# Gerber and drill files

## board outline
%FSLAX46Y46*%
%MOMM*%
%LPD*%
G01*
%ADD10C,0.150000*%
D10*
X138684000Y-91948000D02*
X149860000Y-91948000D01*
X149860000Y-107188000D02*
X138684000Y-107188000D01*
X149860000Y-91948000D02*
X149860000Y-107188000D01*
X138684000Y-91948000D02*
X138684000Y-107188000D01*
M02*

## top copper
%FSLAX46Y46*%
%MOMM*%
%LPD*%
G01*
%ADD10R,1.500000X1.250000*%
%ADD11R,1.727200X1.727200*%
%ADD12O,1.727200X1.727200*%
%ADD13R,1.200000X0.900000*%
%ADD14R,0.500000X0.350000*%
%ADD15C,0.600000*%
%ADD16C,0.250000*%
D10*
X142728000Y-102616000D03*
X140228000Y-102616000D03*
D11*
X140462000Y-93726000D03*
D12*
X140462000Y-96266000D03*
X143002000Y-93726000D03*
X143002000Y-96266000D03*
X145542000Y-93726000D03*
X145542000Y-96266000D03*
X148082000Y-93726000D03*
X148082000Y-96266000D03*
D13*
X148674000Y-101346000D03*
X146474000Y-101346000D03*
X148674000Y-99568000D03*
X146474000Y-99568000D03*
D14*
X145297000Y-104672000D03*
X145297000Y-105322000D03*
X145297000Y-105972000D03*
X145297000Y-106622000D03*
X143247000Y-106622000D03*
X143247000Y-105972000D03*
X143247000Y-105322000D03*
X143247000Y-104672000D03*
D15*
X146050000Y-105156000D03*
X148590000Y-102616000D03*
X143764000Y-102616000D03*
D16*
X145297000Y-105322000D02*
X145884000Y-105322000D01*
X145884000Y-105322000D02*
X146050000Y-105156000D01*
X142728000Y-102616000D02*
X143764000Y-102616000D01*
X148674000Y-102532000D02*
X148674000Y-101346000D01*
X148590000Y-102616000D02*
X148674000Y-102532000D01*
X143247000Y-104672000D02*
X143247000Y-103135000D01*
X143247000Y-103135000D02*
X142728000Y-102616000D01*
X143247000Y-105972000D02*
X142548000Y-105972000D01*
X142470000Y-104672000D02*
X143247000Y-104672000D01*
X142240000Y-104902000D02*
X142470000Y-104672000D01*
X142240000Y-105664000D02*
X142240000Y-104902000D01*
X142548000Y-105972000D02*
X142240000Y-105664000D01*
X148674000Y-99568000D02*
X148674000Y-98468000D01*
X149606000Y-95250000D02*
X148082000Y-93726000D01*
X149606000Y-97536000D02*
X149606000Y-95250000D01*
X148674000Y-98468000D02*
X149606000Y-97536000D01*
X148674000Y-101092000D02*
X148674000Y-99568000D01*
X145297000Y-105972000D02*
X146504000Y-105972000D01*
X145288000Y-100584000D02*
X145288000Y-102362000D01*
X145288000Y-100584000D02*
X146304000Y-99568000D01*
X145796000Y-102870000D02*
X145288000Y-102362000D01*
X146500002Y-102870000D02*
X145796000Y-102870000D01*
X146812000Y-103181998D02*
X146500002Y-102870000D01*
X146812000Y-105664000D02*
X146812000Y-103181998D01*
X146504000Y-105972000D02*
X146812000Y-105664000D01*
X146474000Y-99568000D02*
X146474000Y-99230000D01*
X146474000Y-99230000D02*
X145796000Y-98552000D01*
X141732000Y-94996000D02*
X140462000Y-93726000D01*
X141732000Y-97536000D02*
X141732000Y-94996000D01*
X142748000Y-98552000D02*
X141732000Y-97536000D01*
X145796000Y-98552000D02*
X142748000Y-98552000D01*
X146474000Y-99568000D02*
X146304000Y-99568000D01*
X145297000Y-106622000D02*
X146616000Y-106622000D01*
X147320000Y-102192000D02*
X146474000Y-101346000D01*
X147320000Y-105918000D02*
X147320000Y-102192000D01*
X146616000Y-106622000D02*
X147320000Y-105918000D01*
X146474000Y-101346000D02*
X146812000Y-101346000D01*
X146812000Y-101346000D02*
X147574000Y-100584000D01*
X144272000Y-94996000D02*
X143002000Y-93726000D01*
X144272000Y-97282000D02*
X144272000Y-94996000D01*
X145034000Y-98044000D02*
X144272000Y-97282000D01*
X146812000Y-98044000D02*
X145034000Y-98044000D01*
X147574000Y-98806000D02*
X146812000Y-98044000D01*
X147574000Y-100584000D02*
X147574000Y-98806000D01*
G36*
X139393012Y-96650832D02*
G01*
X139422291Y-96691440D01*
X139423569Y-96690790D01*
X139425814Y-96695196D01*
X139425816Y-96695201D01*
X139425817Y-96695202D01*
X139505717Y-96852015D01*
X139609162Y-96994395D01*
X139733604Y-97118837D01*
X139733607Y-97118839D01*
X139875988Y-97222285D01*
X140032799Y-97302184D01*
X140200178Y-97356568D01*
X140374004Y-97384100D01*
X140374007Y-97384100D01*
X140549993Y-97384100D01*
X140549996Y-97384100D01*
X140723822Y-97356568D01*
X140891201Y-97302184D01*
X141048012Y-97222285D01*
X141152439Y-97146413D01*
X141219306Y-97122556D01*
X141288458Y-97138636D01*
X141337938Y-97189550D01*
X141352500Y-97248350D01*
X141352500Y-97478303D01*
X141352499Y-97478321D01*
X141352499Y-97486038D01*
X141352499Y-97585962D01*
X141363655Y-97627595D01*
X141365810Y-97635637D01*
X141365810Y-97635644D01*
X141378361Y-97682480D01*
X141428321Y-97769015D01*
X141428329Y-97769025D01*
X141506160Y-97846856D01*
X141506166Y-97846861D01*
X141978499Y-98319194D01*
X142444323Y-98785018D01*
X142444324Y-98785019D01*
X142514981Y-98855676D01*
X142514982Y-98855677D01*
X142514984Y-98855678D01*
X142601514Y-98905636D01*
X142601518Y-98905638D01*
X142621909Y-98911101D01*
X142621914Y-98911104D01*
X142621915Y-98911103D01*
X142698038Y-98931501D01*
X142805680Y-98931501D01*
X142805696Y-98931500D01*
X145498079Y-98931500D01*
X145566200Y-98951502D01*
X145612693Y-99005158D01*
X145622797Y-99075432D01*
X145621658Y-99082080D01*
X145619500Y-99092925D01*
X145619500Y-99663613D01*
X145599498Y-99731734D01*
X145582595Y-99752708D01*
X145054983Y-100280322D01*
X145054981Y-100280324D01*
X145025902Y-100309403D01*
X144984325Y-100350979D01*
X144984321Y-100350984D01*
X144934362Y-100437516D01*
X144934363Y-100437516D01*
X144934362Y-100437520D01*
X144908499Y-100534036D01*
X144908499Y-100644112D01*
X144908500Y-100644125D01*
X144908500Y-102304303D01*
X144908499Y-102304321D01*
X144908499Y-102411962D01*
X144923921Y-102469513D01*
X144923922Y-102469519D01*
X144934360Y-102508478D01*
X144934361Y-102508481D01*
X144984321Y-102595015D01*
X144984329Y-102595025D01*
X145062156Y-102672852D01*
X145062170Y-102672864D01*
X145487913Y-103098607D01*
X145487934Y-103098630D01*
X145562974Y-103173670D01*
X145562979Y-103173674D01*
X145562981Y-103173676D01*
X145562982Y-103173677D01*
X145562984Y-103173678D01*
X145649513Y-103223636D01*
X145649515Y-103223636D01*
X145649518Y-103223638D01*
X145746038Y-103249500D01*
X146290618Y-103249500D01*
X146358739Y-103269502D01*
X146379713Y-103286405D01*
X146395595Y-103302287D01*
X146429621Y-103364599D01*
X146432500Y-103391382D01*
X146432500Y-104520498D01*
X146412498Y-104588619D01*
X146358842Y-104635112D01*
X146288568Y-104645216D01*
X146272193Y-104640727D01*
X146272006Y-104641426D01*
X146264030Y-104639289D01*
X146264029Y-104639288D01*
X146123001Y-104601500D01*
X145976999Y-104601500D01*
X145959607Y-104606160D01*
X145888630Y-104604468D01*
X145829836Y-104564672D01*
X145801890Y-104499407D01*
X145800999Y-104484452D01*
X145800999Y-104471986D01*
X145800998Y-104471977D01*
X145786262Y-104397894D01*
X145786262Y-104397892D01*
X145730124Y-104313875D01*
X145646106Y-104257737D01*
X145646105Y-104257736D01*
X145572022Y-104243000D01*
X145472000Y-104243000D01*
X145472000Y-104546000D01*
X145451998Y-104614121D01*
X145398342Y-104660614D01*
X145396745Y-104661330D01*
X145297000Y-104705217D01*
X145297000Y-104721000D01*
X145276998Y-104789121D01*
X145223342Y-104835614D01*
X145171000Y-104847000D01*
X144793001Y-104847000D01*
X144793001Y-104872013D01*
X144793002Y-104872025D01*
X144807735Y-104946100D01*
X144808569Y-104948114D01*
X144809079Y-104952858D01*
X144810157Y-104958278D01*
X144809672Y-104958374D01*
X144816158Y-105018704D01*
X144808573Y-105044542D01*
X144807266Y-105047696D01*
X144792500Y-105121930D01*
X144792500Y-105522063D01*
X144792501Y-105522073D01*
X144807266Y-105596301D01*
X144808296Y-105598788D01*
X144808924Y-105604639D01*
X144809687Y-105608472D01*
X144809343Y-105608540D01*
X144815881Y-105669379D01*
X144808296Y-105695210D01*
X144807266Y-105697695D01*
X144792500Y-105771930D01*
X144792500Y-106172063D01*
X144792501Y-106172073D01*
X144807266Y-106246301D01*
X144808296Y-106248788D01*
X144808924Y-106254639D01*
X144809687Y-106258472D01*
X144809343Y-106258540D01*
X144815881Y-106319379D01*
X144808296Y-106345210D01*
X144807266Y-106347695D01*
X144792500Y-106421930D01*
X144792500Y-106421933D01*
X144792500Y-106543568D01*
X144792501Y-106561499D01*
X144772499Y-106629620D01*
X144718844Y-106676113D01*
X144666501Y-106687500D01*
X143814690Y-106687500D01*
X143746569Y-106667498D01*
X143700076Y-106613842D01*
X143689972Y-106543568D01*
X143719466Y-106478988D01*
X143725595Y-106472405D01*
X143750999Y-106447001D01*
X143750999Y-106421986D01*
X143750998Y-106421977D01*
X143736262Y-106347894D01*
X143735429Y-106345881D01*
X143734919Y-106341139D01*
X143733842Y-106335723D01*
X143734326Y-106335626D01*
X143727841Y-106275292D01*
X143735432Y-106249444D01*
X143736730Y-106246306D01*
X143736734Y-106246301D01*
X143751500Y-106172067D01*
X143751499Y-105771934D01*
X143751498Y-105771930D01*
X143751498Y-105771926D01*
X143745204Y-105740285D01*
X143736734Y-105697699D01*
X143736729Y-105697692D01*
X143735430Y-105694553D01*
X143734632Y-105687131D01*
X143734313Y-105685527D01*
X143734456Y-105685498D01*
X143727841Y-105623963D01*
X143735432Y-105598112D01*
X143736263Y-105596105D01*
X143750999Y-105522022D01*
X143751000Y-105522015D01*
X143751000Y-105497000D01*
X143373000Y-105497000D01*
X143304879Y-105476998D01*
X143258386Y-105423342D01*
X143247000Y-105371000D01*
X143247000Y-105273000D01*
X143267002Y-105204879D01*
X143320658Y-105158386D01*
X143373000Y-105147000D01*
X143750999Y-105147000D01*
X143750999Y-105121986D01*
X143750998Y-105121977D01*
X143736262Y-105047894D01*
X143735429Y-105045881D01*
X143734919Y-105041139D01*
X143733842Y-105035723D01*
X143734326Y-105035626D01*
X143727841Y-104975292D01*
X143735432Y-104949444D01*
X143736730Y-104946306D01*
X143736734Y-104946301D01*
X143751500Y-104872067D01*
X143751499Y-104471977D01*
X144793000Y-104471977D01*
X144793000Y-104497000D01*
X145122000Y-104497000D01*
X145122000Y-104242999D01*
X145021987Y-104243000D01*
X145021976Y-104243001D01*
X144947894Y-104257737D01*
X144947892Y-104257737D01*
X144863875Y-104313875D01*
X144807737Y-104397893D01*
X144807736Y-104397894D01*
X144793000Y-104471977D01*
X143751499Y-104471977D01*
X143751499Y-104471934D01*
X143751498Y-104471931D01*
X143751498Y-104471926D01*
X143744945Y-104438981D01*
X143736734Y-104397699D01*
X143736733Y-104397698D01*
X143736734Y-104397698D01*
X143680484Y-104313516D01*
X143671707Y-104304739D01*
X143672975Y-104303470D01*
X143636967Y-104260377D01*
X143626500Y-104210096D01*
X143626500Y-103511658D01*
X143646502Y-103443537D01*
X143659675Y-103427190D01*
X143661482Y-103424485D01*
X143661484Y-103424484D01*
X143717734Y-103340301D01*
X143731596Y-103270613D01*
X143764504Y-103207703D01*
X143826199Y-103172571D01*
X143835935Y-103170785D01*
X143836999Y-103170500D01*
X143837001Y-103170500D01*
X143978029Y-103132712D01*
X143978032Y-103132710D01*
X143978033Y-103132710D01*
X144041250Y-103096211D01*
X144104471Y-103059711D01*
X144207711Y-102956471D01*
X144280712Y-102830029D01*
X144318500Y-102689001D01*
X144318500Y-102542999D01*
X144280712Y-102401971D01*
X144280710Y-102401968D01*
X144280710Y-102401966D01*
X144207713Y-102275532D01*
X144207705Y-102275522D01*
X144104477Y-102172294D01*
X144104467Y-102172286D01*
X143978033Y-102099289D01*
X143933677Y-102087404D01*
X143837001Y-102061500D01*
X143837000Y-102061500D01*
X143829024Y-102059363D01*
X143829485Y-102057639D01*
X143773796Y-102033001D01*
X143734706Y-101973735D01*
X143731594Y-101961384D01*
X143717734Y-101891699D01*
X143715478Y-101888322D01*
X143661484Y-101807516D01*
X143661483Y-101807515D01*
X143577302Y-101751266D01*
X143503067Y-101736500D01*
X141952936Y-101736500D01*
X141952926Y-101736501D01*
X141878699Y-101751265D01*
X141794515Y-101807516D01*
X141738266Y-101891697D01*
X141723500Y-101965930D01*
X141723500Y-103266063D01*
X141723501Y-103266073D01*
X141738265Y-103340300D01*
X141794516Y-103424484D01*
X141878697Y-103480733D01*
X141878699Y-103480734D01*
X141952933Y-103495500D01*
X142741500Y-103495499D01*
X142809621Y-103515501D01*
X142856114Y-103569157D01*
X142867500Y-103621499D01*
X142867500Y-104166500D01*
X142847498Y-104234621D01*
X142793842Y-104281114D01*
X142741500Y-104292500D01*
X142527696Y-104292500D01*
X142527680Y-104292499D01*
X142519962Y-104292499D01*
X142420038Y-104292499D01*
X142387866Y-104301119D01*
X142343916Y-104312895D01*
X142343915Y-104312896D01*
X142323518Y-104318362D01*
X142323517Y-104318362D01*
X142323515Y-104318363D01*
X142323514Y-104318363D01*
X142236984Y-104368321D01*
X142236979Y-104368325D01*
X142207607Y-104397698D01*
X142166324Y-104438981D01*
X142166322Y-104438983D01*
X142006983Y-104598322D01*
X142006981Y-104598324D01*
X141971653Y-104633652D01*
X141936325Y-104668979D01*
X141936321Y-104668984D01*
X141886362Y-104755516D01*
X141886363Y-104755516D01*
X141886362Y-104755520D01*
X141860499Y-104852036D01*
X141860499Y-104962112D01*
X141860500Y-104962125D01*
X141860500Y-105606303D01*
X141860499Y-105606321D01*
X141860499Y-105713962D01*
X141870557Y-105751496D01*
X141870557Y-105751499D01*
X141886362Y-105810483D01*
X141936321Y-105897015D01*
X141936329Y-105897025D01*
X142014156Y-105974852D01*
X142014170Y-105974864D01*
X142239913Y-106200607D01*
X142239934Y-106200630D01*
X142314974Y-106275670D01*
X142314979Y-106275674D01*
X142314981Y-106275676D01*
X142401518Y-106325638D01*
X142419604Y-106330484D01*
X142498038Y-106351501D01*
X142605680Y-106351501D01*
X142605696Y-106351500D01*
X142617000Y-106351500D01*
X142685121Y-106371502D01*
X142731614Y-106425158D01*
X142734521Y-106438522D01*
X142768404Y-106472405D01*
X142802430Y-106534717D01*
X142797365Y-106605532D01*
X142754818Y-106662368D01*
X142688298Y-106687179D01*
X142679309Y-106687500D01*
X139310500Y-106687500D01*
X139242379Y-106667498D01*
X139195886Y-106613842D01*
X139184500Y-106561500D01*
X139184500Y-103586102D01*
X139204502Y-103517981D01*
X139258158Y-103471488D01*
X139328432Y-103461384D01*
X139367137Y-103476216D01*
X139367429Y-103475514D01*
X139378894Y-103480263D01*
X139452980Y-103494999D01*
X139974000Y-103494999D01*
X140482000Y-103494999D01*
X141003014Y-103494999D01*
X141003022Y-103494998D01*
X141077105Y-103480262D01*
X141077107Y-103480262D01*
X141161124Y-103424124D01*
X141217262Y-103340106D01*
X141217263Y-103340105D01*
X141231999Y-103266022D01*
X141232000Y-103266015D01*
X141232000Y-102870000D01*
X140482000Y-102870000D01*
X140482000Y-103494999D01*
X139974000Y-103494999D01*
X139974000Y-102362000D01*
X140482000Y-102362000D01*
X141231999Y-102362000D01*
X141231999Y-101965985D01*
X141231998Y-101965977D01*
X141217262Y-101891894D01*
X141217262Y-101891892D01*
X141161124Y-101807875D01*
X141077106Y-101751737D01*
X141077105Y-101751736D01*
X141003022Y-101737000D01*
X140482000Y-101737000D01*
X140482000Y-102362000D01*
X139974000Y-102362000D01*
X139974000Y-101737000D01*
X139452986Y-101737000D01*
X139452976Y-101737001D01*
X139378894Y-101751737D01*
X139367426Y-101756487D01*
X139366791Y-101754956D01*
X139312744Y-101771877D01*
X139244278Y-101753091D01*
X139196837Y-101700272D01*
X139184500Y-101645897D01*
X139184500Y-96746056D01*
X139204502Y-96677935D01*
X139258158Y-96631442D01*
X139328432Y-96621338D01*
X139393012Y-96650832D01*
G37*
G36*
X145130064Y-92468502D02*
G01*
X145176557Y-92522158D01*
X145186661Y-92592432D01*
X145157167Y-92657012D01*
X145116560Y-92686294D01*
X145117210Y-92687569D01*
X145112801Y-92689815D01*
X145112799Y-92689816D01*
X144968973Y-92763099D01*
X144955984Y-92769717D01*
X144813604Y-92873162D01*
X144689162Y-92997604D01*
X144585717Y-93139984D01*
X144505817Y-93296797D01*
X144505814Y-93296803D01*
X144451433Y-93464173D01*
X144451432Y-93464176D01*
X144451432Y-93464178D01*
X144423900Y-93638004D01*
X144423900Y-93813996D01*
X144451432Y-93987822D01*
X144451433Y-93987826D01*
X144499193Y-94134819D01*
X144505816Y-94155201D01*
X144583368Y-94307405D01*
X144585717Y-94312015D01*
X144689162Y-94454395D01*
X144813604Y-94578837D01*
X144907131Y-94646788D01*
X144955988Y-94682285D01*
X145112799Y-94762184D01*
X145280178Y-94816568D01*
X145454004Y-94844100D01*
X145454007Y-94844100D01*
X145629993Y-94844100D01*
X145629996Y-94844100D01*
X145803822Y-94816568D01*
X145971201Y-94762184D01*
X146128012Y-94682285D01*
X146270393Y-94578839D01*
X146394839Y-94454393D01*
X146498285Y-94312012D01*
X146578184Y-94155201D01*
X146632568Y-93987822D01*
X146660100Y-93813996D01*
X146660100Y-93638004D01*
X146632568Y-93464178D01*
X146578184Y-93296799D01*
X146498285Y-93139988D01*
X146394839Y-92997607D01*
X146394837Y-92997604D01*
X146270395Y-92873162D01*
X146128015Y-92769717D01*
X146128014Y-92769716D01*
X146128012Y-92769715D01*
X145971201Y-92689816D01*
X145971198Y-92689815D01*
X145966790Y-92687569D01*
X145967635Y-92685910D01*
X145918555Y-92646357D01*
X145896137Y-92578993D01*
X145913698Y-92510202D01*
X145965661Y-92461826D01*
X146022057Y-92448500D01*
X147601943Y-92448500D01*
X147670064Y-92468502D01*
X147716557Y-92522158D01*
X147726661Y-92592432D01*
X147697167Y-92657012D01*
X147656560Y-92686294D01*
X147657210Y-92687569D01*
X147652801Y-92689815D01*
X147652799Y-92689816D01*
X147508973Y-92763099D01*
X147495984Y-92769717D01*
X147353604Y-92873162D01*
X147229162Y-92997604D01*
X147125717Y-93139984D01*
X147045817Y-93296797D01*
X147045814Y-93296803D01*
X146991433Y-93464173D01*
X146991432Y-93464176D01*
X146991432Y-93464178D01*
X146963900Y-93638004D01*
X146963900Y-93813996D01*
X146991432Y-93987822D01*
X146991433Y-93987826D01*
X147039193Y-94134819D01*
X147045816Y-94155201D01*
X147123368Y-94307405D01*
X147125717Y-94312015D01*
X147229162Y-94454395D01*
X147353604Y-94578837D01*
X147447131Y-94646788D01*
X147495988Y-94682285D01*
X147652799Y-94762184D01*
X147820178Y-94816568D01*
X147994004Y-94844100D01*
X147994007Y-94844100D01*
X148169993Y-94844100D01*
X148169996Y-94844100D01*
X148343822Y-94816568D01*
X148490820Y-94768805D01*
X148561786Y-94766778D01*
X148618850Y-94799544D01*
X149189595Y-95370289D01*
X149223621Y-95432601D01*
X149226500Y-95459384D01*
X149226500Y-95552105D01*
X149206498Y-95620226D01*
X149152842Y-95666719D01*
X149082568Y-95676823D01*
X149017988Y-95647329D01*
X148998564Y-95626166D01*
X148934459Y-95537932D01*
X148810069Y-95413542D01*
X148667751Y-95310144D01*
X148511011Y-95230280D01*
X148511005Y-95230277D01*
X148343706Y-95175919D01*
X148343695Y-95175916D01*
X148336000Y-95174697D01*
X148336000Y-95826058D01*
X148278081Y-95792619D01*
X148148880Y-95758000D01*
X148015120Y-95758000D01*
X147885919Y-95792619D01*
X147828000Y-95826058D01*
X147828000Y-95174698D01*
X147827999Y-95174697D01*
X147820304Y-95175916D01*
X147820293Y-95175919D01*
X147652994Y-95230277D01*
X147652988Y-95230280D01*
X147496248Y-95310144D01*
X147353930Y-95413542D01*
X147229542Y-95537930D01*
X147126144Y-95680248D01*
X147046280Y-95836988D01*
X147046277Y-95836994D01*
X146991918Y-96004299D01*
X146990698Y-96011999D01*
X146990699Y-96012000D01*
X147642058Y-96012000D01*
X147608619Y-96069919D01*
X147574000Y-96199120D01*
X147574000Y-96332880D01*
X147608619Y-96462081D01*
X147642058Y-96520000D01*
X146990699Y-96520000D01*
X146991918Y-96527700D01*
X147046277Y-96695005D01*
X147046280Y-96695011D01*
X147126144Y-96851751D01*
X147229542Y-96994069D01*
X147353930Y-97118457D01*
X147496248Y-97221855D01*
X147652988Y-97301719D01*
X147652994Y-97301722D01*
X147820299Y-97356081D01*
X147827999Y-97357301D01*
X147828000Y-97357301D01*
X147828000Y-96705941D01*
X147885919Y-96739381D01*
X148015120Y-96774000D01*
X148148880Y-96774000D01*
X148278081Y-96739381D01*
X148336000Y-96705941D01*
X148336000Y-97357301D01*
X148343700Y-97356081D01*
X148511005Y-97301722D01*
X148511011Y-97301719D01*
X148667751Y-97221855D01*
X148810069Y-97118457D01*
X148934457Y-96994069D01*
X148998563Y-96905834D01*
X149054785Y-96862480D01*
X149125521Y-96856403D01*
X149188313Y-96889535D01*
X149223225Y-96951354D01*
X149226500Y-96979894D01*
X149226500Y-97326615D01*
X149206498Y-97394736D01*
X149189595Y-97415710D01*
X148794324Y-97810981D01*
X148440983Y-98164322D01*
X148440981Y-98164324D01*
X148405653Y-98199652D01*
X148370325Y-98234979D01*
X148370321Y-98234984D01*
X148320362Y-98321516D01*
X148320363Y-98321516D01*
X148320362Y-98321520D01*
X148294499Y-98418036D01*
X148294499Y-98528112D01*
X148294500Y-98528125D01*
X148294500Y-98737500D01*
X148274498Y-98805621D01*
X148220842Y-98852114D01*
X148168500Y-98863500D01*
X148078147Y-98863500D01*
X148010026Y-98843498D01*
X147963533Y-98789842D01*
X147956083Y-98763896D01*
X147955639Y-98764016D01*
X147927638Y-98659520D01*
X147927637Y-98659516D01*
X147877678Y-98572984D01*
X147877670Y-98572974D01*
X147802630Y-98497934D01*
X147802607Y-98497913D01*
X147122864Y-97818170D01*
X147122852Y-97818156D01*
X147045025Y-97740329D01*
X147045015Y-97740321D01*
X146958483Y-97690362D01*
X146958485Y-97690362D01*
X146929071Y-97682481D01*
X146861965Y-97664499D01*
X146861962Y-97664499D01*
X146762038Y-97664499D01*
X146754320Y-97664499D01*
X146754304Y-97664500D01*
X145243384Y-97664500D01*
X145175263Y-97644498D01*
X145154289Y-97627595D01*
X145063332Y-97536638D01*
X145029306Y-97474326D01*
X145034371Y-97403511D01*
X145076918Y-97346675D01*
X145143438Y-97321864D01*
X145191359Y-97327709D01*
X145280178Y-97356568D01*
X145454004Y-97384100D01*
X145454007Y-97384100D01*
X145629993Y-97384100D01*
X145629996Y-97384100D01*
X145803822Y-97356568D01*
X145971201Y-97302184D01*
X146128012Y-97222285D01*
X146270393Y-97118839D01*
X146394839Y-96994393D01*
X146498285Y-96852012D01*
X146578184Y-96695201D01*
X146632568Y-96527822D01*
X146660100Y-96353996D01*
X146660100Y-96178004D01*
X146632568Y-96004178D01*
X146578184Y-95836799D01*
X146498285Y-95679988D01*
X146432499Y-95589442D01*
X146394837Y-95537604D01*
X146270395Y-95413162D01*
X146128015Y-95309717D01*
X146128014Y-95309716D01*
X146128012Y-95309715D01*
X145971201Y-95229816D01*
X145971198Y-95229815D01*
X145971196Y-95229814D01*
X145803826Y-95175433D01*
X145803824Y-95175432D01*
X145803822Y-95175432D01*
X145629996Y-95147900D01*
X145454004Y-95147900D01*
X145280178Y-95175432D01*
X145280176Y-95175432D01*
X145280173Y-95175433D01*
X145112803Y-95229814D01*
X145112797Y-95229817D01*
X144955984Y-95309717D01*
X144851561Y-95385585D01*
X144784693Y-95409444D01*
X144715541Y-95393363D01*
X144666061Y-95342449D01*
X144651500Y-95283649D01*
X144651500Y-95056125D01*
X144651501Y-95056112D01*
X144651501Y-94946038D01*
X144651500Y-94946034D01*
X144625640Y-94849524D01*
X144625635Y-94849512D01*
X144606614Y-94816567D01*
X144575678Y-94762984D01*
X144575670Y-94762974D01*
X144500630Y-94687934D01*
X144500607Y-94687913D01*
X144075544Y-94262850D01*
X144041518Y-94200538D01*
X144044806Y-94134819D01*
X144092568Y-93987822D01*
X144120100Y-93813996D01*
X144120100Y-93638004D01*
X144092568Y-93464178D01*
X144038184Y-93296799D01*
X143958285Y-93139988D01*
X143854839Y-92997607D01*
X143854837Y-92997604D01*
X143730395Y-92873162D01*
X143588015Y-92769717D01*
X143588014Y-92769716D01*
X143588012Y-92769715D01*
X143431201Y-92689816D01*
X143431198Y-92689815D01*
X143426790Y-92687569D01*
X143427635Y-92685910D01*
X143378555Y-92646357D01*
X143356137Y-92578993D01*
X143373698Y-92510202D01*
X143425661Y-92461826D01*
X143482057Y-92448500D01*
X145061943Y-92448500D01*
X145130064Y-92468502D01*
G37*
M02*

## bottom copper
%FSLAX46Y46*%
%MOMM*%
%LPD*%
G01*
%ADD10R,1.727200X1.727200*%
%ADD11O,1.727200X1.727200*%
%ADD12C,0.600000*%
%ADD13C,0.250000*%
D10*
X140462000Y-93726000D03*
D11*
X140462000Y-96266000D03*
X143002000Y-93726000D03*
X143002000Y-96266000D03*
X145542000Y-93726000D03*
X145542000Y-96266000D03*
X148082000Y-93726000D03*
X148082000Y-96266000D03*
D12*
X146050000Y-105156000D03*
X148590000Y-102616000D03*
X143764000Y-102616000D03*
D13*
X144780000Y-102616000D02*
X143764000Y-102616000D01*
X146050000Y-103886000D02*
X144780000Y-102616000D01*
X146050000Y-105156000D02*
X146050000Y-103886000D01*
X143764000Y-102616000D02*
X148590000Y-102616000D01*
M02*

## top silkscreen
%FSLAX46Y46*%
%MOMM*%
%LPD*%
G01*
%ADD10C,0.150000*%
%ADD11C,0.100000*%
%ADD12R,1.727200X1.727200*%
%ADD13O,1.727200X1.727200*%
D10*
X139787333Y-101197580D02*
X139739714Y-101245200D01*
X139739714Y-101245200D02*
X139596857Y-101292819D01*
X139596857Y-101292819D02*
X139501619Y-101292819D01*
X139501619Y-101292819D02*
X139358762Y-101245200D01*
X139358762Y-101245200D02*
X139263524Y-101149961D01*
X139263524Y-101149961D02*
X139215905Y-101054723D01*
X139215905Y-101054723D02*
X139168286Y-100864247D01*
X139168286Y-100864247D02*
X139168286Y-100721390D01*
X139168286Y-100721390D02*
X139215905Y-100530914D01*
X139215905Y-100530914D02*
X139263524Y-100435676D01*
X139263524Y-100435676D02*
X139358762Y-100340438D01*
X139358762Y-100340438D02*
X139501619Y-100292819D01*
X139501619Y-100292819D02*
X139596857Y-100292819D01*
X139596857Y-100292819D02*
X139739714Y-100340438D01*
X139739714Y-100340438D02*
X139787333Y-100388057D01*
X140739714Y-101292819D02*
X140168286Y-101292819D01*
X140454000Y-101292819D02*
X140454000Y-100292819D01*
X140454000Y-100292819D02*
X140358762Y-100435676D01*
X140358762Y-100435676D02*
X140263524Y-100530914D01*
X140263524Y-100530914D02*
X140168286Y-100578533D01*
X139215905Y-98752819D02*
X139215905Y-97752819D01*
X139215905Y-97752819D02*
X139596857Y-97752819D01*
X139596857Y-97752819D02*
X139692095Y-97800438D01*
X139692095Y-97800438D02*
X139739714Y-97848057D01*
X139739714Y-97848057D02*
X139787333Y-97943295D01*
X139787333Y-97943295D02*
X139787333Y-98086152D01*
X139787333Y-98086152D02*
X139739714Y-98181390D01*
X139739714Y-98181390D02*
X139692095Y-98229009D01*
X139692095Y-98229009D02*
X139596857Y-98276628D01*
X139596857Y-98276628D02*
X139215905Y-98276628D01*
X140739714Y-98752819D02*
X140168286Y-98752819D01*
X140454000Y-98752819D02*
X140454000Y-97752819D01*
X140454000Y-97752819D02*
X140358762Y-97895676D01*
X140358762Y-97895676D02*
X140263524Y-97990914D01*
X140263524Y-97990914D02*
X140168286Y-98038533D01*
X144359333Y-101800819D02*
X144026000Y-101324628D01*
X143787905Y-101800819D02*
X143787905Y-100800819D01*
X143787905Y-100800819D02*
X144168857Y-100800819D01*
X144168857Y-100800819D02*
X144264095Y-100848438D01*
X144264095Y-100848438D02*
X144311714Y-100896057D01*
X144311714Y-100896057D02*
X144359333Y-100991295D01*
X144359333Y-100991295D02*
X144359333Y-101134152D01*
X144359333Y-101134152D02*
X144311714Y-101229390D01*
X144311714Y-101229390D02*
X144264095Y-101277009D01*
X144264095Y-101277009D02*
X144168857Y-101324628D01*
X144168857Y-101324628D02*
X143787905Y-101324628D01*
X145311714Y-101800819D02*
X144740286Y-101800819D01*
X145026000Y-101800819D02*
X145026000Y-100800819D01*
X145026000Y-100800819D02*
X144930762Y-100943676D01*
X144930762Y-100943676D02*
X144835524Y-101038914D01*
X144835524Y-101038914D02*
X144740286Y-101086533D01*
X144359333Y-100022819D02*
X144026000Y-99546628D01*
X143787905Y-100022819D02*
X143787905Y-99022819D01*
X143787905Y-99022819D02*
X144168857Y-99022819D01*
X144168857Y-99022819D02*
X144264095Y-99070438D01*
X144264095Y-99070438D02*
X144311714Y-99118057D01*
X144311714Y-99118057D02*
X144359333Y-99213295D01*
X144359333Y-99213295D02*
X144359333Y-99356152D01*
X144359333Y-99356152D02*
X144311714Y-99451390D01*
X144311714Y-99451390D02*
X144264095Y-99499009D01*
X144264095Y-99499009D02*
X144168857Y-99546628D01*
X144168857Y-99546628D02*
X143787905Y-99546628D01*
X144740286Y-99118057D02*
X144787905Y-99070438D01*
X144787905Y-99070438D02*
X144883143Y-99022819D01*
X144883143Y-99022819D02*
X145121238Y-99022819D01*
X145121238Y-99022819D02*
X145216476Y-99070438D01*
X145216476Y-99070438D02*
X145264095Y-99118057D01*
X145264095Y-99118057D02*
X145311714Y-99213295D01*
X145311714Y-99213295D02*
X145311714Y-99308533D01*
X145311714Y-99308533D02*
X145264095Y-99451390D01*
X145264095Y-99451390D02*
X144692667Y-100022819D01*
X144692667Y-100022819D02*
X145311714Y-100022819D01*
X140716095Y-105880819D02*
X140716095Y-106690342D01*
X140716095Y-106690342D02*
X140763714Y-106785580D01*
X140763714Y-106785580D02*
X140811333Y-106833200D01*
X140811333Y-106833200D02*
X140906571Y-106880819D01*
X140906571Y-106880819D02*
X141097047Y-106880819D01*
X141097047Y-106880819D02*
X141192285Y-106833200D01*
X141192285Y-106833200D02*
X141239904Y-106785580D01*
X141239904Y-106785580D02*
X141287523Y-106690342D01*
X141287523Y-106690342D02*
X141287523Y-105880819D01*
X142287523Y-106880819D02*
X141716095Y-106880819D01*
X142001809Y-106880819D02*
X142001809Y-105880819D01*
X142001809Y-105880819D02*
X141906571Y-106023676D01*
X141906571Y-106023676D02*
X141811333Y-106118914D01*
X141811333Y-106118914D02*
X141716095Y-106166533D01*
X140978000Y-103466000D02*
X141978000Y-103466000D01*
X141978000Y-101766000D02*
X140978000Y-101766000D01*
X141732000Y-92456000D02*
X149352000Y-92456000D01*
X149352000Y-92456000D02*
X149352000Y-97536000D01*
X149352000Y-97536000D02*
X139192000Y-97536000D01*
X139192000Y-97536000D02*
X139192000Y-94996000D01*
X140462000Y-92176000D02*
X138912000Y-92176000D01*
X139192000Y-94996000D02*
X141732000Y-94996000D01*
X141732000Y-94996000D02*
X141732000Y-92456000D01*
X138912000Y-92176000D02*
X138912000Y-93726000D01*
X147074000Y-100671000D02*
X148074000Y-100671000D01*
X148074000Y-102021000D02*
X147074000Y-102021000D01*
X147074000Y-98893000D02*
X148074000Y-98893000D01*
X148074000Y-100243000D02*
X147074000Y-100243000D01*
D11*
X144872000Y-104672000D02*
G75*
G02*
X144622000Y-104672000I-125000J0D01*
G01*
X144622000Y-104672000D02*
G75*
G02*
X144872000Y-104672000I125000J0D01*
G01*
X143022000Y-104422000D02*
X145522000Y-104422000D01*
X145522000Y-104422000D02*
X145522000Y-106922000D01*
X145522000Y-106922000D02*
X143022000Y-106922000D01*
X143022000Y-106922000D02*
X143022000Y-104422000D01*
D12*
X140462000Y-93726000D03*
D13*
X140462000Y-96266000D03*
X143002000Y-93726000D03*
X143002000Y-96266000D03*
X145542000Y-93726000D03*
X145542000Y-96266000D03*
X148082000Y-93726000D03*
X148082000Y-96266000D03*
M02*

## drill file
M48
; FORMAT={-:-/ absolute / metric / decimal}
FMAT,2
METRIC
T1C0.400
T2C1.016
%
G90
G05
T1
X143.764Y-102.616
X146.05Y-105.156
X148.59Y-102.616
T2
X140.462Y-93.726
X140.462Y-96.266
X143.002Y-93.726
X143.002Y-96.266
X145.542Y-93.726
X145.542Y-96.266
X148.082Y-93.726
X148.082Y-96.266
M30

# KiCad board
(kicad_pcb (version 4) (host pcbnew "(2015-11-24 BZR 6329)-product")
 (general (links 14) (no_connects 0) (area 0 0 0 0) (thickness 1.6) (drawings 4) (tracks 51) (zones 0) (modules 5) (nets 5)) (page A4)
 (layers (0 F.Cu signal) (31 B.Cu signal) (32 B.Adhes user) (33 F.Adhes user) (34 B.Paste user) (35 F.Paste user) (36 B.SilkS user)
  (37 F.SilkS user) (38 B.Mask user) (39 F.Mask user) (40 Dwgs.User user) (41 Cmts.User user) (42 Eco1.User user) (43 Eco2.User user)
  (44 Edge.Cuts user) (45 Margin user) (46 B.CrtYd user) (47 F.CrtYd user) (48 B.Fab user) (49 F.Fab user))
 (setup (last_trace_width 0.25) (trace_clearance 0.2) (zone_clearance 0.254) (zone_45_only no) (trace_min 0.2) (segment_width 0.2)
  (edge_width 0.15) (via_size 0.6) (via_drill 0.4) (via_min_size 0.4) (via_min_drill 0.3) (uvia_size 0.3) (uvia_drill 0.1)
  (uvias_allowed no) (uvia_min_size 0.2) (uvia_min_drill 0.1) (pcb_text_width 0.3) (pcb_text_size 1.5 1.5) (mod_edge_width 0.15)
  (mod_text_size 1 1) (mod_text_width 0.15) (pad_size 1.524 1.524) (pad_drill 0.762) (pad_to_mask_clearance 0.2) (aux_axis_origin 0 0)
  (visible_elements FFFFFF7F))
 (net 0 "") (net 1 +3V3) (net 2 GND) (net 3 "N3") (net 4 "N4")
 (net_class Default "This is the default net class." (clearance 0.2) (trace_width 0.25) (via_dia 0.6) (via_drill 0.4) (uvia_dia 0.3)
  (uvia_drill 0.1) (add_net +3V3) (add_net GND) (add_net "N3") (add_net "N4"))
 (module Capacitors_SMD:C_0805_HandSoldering (layer F.Cu) (at 141.478 102.616 180)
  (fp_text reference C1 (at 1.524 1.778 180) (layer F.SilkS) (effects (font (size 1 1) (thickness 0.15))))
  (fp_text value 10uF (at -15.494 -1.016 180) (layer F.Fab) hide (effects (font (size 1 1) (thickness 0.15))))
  (fp_line (start 0.5 -0.85) (end -0.5 -0.85) (layer F.SilkS) (width 0.15))
  (fp_line (start -0.5 0.85) (end 0.5 0.85) (layer F.SilkS) (width 0.15))
  (pad 1 smd rect (at -1.25 0 180) (size 1.5 1.25) (layers F.Cu F.Paste F.Mask) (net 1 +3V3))
  (pad 2 smd rect (at 1.25 0 180) (size 1.5 1.25) (layers F.Cu F.Paste F.Mask) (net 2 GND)))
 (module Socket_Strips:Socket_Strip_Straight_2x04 (layer F.Cu) (at 140.462 93.726)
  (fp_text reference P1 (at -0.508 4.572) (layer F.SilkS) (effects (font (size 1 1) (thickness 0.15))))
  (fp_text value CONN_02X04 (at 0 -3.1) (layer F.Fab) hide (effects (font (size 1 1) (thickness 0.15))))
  (fp_line (start 1.27 -1.27) (end 8.89 -1.27) (layer F.SilkS) (width 0.15))
  (fp_line (start 8.89 -1.27) (end 8.89 3.81) (layer F.SilkS) (width 0.15))
  (fp_line (start 8.89 3.81) (end -1.27 3.81) (layer F.SilkS) (width 0.15))
  (fp_line (start -1.27 3.81) (end -1.27 1.27) (layer F.SilkS) (width 0.15))
  (fp_line (start 0 -1.55) (end -1.55 -1.55) (layer F.SilkS) (width 0.15))
  (fp_line (start -1.27 1.27) (end 1.27 1.27) (layer F.SilkS) (width 0.15))
  (fp_line (start 1.27 1.27) (end 1.27 -1.27) (layer F.SilkS) (width 0.15))
  (fp_line (start -1.55 -1.55) (end -1.55 0) (layer F.SilkS) (width 0.15))
  (pad 1 thru_hole rect (at 0 0) (size 1.7272 1.7272) (drill 1.016) (layers *.Cu *.Mask F.SilkS) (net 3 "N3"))
  (pad 2 thru_hole oval (at 0 2.54) (size 1.7272 1.7272) (drill 1.016) (layers *.Cu *.Mask F.SilkS))
  (pad 3 thru_hole oval (at 2.54 0) (size 1.7272 1.7272) (drill 1.016) (layers *.Cu *.Mask F.SilkS) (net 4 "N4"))
  (pad 4 thru_hole oval (at 2.54 2.54) (size 1.7272 1.7272) (drill 1.016) (layers *.Cu *.Mask F.SilkS))
  (pad 5 thru_hole oval (at 5.08 0) (size 1.7272 1.7272) (drill 1.016) (layers *.Cu *.Mask F.SilkS))
  (pad 6 thru_hole oval (at 5.08 2.54) (size 1.7272 1.7272) (drill 1.016) (layers *.Cu *.Mask F.SilkS))
  (pad 7 thru_hole oval (at 7.62 0) (size 1.7272 1.7272) (drill 1.016) (layers *.Cu *.Mask F.SilkS) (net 1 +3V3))
  (pad 8 thru_hole oval (at 7.62 2.54) (size 1.7272 1.7272) (drill 1.016) (layers *.Cu *.Mask F.SilkS) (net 2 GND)))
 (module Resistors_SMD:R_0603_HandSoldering (layer F.Cu) (at 147.574 101.346 180)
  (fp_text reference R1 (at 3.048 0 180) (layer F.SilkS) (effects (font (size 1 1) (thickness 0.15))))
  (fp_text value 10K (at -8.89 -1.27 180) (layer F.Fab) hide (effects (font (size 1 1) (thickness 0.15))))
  (fp_line (start 0.5 0.675) (end -0.5 0.675) (layer F.SilkS) (width 0.15))
  (fp_line (start -0.5 -0.675) (end 0.5 -0.675) (layer F.SilkS) (width 0.15))
  (pad 1 smd rect (at -1.1 0 180) (size 1.2 0.9) (layers F.Cu F.Paste F.Mask) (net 1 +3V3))
  (pad 2 smd rect (at 1.1 0 180) (size 1.2 0.9) (layers F.Cu F.Paste F.Mask) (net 4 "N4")))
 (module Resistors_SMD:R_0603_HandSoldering (layer F.Cu) (at 147.574 99.568 180)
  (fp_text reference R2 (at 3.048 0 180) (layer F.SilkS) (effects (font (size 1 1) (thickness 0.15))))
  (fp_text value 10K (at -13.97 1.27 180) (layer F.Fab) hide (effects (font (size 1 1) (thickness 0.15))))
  (fp_line (start 0.5 0.675) (end -0.5 0.675) (layer F.SilkS) (width 0.15))
  (fp_line (start -0.5 -0.675) (end 0.5 -0.675) (layer F.SilkS) (width 0.15))
  (pad 1 smd rect (at -1.1 0 180) (size 1.2 0.9) (layers F.Cu F.Paste F.Mask) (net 1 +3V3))
  (pad 2 smd rect (at 1.1 0 180) (size 1.2 0.9) (layers F.Cu F.Paste F.Mask) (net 3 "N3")))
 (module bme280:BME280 (layer F.Cu) (at 144.272 106.172)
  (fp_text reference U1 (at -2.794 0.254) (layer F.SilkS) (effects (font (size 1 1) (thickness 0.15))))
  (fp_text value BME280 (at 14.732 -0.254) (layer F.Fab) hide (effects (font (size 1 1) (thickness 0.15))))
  (fp_circle (center 0.475 -1.5) (end 0.55 -1.4) (layer F.SilkS) (width 0.1))
  (fp_line (start -1.25 -1.75) (end 1.25 -1.75) (layer F.SilkS) (width 0.1))
  (fp_line (start 1.25 -1.75) (end 1.25 0.75) (layer F.SilkS) (width 0.1))
  (fp_line (start 1.25 0.75) (end -1.25 0.75) (layer F.SilkS) (width 0.1))
  (fp_line (start -1.25 0.75) (end -1.25 -1.75) (layer F.SilkS) (width 0.1))
  (pad 1 smd rect (at 1.025 -1.5) (size 0.5 0.35) (layers F.Cu F.Paste F.Mask) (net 2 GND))
  (pad 2 smd rect (at 1.025 -0.85) (size 0.5 0.35) (layers F.Cu F.Paste F.Mask) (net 1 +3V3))
  (pad 3 smd rect (at 1.025 -0.2) (size 0.5 0.35) (layers F.Cu F.Paste F.Mask) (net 3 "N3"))
  (pad 4 smd rect (at 1.025 0.45) (size 0.5 0.35) (layers F.Cu F.Paste F.Mask) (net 4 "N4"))
  (pad 5 smd rect (at -1.025 0.45) (size 0.5 0.35) (layers F.Cu F.Paste F.Mask) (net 2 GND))
  (pad 6 smd rect (at -1.025 -0.2) (size 0.5 0.35) (layers F.Cu F.Paste F.Mask) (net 1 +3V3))
  (pad 7 smd rect (at -1.025 -0.85) (size 0.5 0.35) (layers F.Cu F.Paste F.Mask) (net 2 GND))
  (pad 8 smd rect (at -1.025 -1.5) (size 0.5 0.35) (layers F.Cu F.Paste F.Mask) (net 1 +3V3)))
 (gr_line (start 138.684 91.948) (end 149.86 91.948) (angle 90) (layer Edge.Cuts) (width 0.15))
 (gr_line (start 149.86 107.188) (end 138.684 107.188) (angle 90) (layer Edge.Cuts) (width 0.15))
 (gr_line (start 149.86 91.948) (end 149.86 107.188) (angle 90) (layer Edge.Cuts) (width 0.15))
 (gr_line (start 138.684 91.948) (end 138.684 107.188) (angle 90) (layer Edge.Cuts) (width 0.15))
 (segment (start 145.297 105.322) (end 145.884 105.322) (width 0.25) (layer F.Cu) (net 1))
 (segment (start 144.78 102.616) (end 143.764 102.616) (width 0.25) (layer B.Cu) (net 1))
 (segment (start 146.05 103.886) (end 144.78 102.616) (width 0.25) (layer B.Cu) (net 1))
 (segment (start 146.05 105.156) (end 146.05 103.886) (width 0.25) (layer B.Cu) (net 1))
 (via (at 146.05 105.156) (size 0.6) (drill 0.4) (layers F.Cu B.Cu) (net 1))
 (segment (start 145.884 105.322) (end 146.05 105.156) (width 0.25) (layer F.Cu) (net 1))
 (segment (start 142.728 102.616) (end 143.764 102.616) (width 0.25) (layer F.Cu) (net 1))
 (segment (start 148.674 102.532) (end 148.674 101.346) (width 0.25) (layer F.Cu) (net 1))
 (segment (start 148.59 102.616) (end 148.674 102.532) (width 0.25) (layer F.Cu) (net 1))
 (via (at 148.59 102.616) (size 0.6) (drill 0.4) (layers F.Cu B.Cu) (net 1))
 (segment (start 143.764 102.616) (end 148.59 102.616) (width 0.25) (layer B.Cu) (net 1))
 (via (at 143.764 102.616) (size 0.6) (drill 0.4) (layers F.Cu B.Cu) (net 1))
 (segment (start 143.247 104.672) (end 143.247 103.135) (width 0.25) (layer F.Cu) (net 1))
 (segment (start 143.247 103.135) (end 142.728 102.616) (width 0.25) (layer F.Cu) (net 1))
 (segment (start 143.247 105.972) (end 142.548 105.972) (width 0.25) (layer F.Cu) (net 1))
 (segment (start 142.47 104.672) (end 143.247 104.672) (width 0.25) (layer F.Cu) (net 1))
 (segment (start 142.24 104.902) (end 142.47 104.672) (width 0.25) (layer F.Cu) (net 1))
 (segment (start 142.24 105.664) (end 142.24 104.902) (width 0.25) (layer F.Cu) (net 1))
 (segment (start 142.548 105.972) (end 142.24 105.664) (width 0.25) (layer F.Cu) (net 1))
 (segment (start 148.674 99.568) (end 148.674 98.468) (width 0.25) (layer F.Cu) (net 1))
 (segment (start 149.606 95.25) (end 148.082 93.726) (width 0.25) (layer F.Cu) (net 1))
 (segment (start 149.606 97.536) (end 149.606 95.25) (width 0.25) (layer F.Cu) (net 1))
 (segment (start 148.674 98.468) (end 149.606 97.536) (width 0.25) (layer F.Cu) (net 1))
 (segment (start 148.674 101.092) (end 148.674 99.568) (width 0.25) (layer F.Cu) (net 1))
 (segment (start 145.297 105.972) (end 146.504 105.972) (width 0.25) (layer F.Cu) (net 3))
 (segment (start 145.288 100.584) (end 145.288 102.362) (width 0.25) (layer F.Cu) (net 3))
 (segment (start 145.288 100.584) (end 146.304 99.568) (width 0.25) (layer F.Cu) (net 3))
 (segment (start 145.796 102.87) (end 145.288 102.362) (width 0.25) (layer F.Cu) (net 3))
 (segment (start 146.500002 102.87) (end 145.796 102.87) (width 0.25) (layer F.Cu) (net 3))
 (segment (start 146.812 103.181998) (end 146.500002 102.87) (width 0.25) (layer F.Cu) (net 3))
 (segment (start 146.812 105.664) (end 146.812 103.181998) (width 0.25) (layer F.Cu) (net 3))
 (segment (start 146.504 105.972) (end 146.812 105.664) (width 0.25) (layer F.Cu) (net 3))
 (segment (start 146.474 99.568) (end 146.474 99.23) (width 0.25) (layer F.Cu) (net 3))
 (segment (start 146.474 99.23) (end 145.796 98.552) (width 0.25) (layer F.Cu) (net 3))
 (segment (start 141.732 94.996) (end 140.462 93.726) (width 0.25) (layer F.Cu) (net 3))
 (segment (start 141.732 97.536) (end 141.732 94.996) (width 0.25) (layer F.Cu) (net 3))
 (segment (start 142.748 98.552) (end 141.732 97.536) (width 0.25) (layer F.Cu) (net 3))
 (segment (start 145.796 98.552) (end 142.748 98.552) (width 0.25) (layer F.Cu) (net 3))
 (segment (start 146.474 99.568) (end 146.304 99.568) (width 0.25) (layer F.Cu) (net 3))
 (segment (start 145.297 106.622) (end 146.616 106.622) (width 0.25) (layer F.Cu) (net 4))
 (segment (start 147.32 102.192) (end 146.474 101.346) (width 0.25) (layer F.Cu) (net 4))
 (segment (start 147.32 105.918) (end 147.32 102.192) (width 0.25) (layer F.Cu) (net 4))
 (segment (start 146.616 106.622) (end 147.32 105.918) (width 0.25) (layer F.Cu) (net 4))
 (segment (start 146.474 101.346) (end 146.812 101.346) (width 0.25) (layer F.Cu) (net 4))
 (segment (start 146.812 101.346) (end 147.574 100.584) (width 0.25) (layer F.Cu) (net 4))
 (segment (start 144.272 94.996) (end 143.002 93.726) (width 0.25) (layer F.Cu) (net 4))
 (segment (start 144.272 97.282) (end 144.272 94.996) (width 0.25) (layer F.Cu) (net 4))
 (segment (start 145.034 98.044) (end 144.272 97.282) (width 0.25) (layer F.Cu) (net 4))
 (segment (start 146.812 98.044) (end 145.034 98.044) (width 0.25) (layer F.Cu) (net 4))
 (segment (start 147.574 98.806) (end 146.812 98.044) (width 0.25) (layer F.Cu) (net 4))
 (segment (start 147.574 100.584) (end 147.574 98.806) (width 0.25) (layer F.Cu) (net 4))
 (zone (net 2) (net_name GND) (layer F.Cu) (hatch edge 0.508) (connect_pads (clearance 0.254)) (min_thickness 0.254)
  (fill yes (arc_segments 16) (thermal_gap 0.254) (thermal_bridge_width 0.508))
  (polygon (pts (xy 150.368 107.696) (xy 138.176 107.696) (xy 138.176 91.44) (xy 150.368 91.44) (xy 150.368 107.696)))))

